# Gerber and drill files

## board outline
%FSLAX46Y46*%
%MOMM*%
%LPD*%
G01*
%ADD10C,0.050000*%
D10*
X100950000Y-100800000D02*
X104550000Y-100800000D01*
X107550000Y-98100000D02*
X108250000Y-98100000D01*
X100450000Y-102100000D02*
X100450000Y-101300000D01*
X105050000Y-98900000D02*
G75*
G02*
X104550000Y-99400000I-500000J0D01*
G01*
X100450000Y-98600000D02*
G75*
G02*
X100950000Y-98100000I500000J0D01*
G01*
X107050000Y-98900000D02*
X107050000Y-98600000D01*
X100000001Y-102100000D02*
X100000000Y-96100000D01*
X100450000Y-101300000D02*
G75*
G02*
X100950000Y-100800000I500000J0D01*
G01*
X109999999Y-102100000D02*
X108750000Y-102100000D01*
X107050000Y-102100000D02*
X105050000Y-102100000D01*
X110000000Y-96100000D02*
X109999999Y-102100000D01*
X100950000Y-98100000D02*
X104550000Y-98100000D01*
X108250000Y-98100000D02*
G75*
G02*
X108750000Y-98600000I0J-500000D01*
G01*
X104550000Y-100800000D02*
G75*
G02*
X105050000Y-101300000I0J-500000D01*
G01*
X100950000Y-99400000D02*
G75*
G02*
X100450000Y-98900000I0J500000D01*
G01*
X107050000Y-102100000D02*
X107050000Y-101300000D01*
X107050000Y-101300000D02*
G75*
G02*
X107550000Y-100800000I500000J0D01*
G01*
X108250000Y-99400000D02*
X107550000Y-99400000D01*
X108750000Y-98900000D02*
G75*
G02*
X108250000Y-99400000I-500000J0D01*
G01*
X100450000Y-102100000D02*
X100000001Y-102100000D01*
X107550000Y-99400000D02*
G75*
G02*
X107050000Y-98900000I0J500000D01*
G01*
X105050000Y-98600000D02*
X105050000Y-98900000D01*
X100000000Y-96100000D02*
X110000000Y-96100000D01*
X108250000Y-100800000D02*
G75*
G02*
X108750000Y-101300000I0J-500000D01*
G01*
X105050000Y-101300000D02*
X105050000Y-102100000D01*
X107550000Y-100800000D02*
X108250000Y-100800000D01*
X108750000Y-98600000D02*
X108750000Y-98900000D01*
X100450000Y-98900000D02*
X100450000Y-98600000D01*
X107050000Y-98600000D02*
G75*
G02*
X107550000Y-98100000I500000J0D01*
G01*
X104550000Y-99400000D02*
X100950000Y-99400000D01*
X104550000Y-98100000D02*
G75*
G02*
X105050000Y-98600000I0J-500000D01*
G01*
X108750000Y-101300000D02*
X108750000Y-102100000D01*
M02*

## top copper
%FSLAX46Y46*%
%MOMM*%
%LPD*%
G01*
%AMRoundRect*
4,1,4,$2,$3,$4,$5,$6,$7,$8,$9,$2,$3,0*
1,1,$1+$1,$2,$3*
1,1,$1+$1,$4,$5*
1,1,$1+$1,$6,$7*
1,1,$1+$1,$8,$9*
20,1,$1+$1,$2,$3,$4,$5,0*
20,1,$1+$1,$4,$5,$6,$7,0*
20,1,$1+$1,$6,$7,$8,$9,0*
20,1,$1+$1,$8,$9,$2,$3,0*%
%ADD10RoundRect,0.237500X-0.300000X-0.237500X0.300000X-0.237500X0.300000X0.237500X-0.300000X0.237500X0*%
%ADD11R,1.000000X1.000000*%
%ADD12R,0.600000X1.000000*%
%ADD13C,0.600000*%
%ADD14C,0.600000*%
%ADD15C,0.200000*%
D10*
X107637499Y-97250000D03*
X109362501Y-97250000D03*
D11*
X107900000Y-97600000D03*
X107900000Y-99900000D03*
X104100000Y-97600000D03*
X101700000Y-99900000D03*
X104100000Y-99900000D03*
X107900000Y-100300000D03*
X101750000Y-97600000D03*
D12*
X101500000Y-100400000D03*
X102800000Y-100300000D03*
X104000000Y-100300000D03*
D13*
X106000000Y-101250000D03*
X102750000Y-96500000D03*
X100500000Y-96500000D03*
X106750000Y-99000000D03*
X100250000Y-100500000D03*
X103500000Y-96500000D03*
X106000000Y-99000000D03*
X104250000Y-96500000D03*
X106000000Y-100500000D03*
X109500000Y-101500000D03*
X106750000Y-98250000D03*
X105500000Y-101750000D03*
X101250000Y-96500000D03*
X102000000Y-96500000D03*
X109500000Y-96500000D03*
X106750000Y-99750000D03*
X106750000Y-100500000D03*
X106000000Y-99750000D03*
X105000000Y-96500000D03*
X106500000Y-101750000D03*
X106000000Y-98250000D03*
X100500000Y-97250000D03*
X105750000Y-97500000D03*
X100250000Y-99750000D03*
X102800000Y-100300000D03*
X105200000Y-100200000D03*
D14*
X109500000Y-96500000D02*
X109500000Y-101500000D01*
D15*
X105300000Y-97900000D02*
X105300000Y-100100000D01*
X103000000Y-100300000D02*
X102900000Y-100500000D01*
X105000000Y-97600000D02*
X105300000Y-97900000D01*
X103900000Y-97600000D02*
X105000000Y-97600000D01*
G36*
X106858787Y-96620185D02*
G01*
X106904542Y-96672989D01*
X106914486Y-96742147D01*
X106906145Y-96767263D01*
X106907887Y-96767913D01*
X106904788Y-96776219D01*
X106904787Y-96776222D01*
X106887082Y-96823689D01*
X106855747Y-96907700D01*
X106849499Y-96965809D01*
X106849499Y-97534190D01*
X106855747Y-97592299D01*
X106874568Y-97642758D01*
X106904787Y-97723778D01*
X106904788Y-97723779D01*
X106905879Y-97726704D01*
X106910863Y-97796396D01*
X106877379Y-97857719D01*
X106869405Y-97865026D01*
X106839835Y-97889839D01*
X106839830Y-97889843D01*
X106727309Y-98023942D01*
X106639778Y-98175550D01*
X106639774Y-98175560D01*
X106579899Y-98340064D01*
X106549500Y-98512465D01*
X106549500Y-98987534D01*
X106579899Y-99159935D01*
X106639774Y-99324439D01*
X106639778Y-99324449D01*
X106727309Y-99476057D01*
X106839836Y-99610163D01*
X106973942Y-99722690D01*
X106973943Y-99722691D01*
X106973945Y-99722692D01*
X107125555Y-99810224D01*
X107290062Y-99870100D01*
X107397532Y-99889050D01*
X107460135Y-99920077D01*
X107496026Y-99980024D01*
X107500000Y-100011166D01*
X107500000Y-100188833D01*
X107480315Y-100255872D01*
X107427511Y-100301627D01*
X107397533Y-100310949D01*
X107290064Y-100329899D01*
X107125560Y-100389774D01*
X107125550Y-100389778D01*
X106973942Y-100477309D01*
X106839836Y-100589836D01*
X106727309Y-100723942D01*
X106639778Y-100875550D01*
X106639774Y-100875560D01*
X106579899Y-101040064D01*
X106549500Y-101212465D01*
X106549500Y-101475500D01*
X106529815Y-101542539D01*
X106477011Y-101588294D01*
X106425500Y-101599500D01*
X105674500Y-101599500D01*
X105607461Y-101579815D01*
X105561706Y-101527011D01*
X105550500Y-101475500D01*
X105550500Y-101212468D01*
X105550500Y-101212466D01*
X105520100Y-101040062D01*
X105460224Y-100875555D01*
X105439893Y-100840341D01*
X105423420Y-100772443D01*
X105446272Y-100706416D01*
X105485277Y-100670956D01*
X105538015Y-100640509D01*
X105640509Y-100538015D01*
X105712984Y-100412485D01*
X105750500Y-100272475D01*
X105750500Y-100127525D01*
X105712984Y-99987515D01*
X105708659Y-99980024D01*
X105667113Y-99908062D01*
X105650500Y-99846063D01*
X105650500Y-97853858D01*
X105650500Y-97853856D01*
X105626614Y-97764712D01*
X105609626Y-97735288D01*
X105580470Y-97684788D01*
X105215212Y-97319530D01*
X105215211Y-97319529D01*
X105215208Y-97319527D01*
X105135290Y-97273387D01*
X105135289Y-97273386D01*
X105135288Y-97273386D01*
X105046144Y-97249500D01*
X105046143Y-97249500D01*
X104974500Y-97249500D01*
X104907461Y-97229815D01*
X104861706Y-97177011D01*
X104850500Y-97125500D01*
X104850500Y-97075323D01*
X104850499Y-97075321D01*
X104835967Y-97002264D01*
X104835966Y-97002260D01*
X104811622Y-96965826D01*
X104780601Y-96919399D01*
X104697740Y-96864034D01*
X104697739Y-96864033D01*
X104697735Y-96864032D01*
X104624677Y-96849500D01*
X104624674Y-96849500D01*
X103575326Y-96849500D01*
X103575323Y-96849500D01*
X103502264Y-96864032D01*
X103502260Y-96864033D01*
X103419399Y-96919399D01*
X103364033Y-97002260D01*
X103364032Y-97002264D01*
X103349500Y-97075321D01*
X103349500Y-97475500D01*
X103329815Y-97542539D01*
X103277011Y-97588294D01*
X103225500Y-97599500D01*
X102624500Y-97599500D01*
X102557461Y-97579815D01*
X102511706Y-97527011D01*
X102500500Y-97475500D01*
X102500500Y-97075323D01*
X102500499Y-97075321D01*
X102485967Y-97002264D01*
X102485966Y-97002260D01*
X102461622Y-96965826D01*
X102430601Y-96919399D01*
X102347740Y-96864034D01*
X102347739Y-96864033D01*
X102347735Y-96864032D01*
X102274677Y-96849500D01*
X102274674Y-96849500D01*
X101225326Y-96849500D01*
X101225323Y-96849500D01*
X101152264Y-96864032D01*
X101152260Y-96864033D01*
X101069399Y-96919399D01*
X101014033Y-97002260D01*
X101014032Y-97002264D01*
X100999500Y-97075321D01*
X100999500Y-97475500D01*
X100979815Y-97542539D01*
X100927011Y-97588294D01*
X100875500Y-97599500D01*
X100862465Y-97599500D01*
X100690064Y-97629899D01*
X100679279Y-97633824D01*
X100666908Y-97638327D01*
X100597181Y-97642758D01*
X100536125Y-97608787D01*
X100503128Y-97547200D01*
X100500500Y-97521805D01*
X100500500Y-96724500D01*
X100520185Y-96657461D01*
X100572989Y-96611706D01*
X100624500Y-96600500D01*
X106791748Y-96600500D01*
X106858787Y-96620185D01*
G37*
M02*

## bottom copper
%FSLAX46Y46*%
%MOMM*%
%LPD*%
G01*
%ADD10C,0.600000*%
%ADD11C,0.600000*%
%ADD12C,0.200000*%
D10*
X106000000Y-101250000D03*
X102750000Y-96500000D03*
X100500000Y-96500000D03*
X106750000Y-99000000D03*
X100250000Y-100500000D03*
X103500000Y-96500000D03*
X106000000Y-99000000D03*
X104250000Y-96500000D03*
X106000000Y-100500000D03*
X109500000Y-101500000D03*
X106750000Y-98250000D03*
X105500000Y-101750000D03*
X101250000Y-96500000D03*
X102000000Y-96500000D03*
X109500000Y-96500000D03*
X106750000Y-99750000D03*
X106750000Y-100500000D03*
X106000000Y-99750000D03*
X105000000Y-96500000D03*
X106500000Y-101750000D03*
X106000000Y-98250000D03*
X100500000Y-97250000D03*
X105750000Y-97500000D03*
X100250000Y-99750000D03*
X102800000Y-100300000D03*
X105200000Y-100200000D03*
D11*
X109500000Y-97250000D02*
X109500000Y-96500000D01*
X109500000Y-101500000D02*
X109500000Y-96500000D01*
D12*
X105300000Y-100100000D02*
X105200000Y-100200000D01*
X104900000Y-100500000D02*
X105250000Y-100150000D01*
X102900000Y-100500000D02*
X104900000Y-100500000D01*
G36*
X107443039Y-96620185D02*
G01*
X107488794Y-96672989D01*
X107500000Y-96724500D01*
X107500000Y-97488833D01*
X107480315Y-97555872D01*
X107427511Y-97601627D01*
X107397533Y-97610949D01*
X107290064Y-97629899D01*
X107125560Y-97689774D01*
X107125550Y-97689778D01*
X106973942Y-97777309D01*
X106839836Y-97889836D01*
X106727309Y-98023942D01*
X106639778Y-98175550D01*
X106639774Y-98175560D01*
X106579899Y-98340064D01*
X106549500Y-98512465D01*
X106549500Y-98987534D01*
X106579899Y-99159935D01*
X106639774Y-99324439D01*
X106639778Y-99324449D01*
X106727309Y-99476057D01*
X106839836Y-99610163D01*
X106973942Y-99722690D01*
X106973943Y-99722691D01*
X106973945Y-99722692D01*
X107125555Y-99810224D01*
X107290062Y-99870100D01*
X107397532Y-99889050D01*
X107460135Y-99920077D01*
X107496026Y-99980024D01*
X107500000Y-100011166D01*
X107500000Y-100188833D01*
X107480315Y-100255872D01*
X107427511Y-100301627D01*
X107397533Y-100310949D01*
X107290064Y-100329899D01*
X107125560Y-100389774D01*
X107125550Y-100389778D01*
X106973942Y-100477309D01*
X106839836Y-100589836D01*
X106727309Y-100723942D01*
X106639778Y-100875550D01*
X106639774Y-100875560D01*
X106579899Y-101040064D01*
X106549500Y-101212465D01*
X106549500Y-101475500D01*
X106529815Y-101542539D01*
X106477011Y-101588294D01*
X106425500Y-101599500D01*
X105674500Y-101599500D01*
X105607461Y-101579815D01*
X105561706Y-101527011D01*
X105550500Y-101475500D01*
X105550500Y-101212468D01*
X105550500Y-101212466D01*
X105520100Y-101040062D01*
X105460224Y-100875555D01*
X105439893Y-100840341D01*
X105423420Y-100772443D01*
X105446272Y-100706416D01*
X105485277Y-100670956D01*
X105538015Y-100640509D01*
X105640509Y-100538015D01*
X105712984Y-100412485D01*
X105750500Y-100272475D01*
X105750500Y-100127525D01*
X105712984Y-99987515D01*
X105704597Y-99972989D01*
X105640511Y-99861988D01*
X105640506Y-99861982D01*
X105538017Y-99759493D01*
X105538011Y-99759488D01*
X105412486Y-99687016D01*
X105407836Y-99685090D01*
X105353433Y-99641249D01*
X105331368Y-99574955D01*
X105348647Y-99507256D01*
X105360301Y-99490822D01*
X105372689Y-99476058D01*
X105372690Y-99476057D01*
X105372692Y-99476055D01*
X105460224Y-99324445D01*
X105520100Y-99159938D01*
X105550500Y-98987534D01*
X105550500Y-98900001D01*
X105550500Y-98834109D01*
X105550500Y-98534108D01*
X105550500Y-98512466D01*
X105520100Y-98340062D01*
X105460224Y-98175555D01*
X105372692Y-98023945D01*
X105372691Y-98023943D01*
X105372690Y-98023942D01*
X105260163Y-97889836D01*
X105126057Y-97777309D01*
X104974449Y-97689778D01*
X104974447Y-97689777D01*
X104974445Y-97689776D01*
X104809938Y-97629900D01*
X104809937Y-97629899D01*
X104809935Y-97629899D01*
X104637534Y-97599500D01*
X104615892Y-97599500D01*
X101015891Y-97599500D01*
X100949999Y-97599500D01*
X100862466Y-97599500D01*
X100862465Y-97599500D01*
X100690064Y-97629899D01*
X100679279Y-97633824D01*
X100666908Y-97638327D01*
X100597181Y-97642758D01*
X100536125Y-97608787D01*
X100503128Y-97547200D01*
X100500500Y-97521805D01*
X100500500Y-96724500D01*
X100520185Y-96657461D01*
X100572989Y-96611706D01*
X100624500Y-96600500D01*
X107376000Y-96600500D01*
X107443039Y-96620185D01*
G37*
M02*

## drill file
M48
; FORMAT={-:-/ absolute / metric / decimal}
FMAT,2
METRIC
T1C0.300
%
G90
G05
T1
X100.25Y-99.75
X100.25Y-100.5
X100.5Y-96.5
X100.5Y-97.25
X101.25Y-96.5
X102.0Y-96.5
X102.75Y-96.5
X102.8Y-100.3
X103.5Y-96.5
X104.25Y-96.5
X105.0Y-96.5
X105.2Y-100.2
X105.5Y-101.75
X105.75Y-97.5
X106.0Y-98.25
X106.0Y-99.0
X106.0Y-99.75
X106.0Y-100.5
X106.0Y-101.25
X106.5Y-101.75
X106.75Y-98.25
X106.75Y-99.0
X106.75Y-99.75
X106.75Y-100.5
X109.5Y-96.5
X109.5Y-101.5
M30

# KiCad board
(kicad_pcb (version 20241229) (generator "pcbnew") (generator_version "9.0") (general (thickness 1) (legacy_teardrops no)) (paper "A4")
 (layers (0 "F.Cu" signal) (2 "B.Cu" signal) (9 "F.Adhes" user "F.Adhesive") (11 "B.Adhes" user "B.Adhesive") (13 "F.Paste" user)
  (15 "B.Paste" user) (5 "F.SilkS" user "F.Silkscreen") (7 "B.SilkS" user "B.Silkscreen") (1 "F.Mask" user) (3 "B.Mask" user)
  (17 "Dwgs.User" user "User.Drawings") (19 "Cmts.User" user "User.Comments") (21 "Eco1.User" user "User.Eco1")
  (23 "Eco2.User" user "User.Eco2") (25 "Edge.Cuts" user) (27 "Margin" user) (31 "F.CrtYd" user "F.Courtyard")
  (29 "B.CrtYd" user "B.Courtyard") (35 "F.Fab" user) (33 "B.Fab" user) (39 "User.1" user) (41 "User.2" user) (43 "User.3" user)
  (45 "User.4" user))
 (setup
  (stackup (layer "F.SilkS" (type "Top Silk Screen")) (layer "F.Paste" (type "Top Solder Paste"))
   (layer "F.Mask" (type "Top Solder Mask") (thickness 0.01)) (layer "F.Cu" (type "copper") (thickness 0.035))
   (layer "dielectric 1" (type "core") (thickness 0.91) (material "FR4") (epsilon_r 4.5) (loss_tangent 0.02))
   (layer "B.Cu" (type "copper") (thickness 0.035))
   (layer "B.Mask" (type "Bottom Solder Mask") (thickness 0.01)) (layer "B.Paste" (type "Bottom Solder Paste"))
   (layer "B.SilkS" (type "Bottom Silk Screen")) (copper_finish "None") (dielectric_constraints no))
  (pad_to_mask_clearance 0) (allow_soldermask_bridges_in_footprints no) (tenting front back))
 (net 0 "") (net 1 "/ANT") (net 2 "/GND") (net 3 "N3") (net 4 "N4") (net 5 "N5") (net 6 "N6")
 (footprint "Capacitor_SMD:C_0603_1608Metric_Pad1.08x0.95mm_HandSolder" (layer "F.Cu") (at 108.5 97.25)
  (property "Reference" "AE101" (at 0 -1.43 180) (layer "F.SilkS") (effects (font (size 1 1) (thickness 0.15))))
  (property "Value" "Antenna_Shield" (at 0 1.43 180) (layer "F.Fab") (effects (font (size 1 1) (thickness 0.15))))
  (pad "1" smd roundrect (at -0.862501 0) (size 1.075 0.95) (layers "F.Cu" "F.Mask" "F.Paste") (roundrect_rratio 0.25) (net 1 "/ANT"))
  (pad "2" smd roundrect (at 0.862501 0) (size 1.075 0.95) (layers "F.Cu" "F.Mask" "F.Paste") (roundrect_rratio 0.25) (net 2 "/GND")))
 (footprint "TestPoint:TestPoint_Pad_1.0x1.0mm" (layer "F.Cu") (at 107.9 97.6)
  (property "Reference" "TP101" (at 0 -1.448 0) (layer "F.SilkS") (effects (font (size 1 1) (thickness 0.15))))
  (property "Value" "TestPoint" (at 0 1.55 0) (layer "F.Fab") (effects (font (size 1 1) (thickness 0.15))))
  (pad "1" smd rect (at 0 0) (size 1 1) (layers "F.Cu" "F.Mask") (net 1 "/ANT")))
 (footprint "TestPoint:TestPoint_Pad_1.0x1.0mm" (layer "F.Cu") (at 107.9 99.9)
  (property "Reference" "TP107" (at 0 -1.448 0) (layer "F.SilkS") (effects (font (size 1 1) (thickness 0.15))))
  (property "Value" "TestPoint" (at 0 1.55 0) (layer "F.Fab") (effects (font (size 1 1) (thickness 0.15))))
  (pad "1" smd rect (at 0 0) (size 1 1) (layers "F.Cu" "F.Mask") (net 2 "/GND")))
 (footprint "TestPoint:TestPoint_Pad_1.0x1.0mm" (layer "F.Cu") (at 104.1 97.6 -90)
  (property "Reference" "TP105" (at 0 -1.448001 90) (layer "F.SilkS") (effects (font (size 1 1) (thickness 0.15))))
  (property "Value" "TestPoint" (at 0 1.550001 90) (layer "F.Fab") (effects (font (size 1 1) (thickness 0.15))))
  (pad "1" smd rect (at 0 0 270) (size 1 1) (layers "F.Cu" "F.Mask") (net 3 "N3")))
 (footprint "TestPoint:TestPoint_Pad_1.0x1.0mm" (layer "F.Cu") (at 101.7 99.9)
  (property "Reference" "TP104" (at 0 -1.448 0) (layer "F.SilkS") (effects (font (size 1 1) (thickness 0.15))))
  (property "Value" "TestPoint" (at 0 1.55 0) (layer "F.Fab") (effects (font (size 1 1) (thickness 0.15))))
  (pad "1" smd rect (at 0 0) (size 1 1) (layers "F.Cu" "F.Mask") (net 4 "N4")))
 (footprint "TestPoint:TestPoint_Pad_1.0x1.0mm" (layer "F.Cu") (at 104.1 99.9)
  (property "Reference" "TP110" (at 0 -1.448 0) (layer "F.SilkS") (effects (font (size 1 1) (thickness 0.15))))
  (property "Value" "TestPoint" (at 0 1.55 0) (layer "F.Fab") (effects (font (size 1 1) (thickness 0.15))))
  (pad "1" smd rect (at 0 0) (size 1 1) (layers "F.Cu" "F.Mask") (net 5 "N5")))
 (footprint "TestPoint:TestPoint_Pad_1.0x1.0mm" (layer "F.Cu") (at 107.9 100.3)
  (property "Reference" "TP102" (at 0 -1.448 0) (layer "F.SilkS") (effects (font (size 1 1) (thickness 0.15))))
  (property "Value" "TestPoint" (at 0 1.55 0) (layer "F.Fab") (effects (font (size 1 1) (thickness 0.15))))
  (pad "1" smd rect (at 0 0) (size 1 1) (layers "F.Cu" "F.Mask") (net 2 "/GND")))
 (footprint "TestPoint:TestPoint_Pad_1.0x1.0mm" (layer "F.Cu") (at 101.7 97.6)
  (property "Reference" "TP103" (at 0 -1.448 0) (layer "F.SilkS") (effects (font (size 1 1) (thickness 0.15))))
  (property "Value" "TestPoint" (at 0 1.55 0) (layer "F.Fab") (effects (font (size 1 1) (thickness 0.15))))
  (pad "1" smd rect (at 0.05 0) (size 1 1) (layers "F.Cu" "F.Mask") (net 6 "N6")))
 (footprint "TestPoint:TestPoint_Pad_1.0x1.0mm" (layer "F.Cu") (at 101.5 100.4)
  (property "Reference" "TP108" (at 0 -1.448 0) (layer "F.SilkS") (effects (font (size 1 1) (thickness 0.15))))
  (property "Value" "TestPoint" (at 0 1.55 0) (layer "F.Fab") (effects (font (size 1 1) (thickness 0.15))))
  (pad "1" smd rect (at 0 0) (size 0.6 1) (layers "F.Cu" "F.Mask") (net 4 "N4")))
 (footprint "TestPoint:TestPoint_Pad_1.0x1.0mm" (layer "F.Cu") (at 102.7 100.3)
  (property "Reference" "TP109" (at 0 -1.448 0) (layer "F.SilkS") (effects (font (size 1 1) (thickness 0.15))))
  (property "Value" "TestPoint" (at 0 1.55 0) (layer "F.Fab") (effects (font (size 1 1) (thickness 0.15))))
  (pad "1" smd rect (at 0.1 0) (size 0.6 1) (layers "F.Cu" "F.Mask") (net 3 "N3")))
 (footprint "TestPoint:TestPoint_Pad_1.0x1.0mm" (layer "F.Cu") (at 104 100.3)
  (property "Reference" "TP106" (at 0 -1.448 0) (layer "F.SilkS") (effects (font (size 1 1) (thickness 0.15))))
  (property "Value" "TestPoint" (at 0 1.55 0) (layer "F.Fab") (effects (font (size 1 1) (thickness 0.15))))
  (pad "1" smd rect (at 0 0) (size 0.6 1) (layers "F.Cu" "F.Mask") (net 5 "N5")))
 (gr_line (start 100.95 100.8) (end 104.55 100.8) (stroke (width 0.05) (type default)) (layer "Edge.Cuts"))
 (gr_line (start 107.55 98.1) (end 108.25 98.1) (stroke (width 0.05) (type default)) (layer "Edge.Cuts"))
 (gr_line (start 100.45 102.1) (end 100.45 101.3) (stroke (width 0.05) (type default)) (layer "Edge.Cuts"))
 (gr_arc (start 105.05 98.9) (mid 104.903553 99.253553) (end 104.55 99.4) (stroke (width 0.05) (type default)) (layer "Edge.Cuts"))
 (gr_arc (start 100.45 98.6) (mid 100.596447 98.246447) (end 100.95 98.1) (stroke (width 0.05) (type default)) (layer "Edge.Cuts"))
 (gr_line (start 107.05 98.9) (end 107.05 98.6) (stroke (width 0.05) (type default)) (layer "Edge.Cuts"))
 (gr_line (start 100.000001 102.1) (end 100 96.1) (stroke (width 0.05) (type default)) (layer "Edge.Cuts"))
 (gr_arc (start 100.45 101.3) (mid 100.596447 100.946447) (end 100.95 100.8) (stroke (width 0.05) (type default)) (layer "Edge.Cuts"))
 (gr_line (start 109.999999 102.1) (end 108.75 102.1) (stroke (width 0.05) (type default)) (layer "Edge.Cuts"))
 (gr_line (start 107.05 102.1) (end 105.05 102.1) (stroke (width 0.05) (type default)) (layer "Edge.Cuts"))
 (gr_line (start 110 96.1) (end 109.999999 102.1) (stroke (width 0.05) (type default)) (layer "Edge.Cuts"))
 (gr_line (start 100.95 98.1) (end 104.55 98.1) (stroke (width 0.05) (type default)) (layer "Edge.Cuts"))
 (gr_arc (start 108.25 98.1) (mid 108.603553 98.246447) (end 108.75 98.6) (stroke (width 0.05) (type default)) (layer "Edge.Cuts"))
 (gr_arc (start 104.55 100.8) (mid 104.903553 100.946447) (end 105.05 101.3) (stroke (width 0.05) (type default)) (layer "Edge.Cuts"))
 (gr_arc (start 100.95 99.4) (mid 100.596447 99.253553) (end 100.45 98.9) (stroke (width 0.05) (type default)) (layer "Edge.Cuts"))
 (gr_line (start 107.05 102.1) (end 107.05 101.3) (stroke (width 0.05) (type default)) (layer "Edge.Cuts"))
 (gr_arc (start 107.05 101.3) (mid 107.196447 100.946447) (end 107.55 100.8) (stroke (width 0.05) (type default)) (layer "Edge.Cuts"))
 (gr_line (start 108.25 99.4) (end 107.55 99.4) (stroke (width 0.05) (type default)) (layer "Edge.Cuts"))
 (gr_arc (start 108.75 98.9) (mid 108.603553 99.253553) (end 108.25 99.4) (stroke (width 0.05) (type default)) (layer "Edge.Cuts"))
 (gr_line (start 100.45 102.1) (end 100.000001 102.1) (stroke (width 0.05) (type default)) (layer "Edge.Cuts"))
 (gr_arc (start 107.55 99.4) (mid 107.196447 99.253553) (end 107.05 98.9) (stroke (width 0.05) (type default)) (layer "Edge.Cuts"))
 (gr_line (start 105.05 98.6) (end 105.05 98.9) (stroke (width 0.05) (type default)) (layer "Edge.Cuts"))
 (gr_line (start 100 96.1) (end 110 96.1) (stroke (width 0.05) (type default)) (layer "Edge.Cuts"))
 (gr_arc (start 108.25 100.8) (mid 108.603553 100.946447) (end 108.75 101.3) (stroke (width 0.05) (type default)) (layer "Edge.Cuts"))
 (gr_line (start 105.05 101.3) (end 105.05 102.1) (stroke (width 0.05) (type default)) (layer "Edge.Cuts"))
 (gr_line (start 107.55 100.8) (end 108.25 100.8) (stroke (width 0.05) (type default)) (layer "Edge.Cuts"))
 (gr_line (start 108.75 98.6) (end 108.75 98.9) (stroke (width 0.05) (type default)) (layer "Edge.Cuts"))
 (gr_line (start 100.45 98.9) (end 100.45 98.6) (stroke (width 0.05) (type default)) (layer "Edge.Cuts"))
 (gr_arc (start 107.05 98.6) (mid 107.196447 98.246447) (end 107.55 98.1) (stroke (width 0.05) (type default)) (layer "Edge.Cuts"))
 (gr_line (start 104.55 99.4) (end 100.95 99.4) (stroke (width 0.05) (type default)) (layer "Edge.Cuts"))
 (gr_arc (start 104.55 98.1) (mid 104.903553 98.246447) (end 105.05 98.6) (stroke (width 0.05) (type default)) (layer "Edge.Cuts"))
 (gr_line (start 108.75 101.3) (end 108.75 102.1) (stroke (width 0.05) (type default)) (layer "Edge.Cuts"))
 (segment (start 109.5 96.5) (end 109.5 101.5) (width 0.6) (layer "F.Cu") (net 2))
 (via (at 106 101.25) (size 0.6) (drill 0.3) (layers "F.Cu" "B.Cu") (free yes) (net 2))
 (via (at 102.75 96.5) (size 0.6) (drill 0.3) (layers "F.Cu" "B.Cu") (free yes) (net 2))
 (via (at 100.5 96.5) (size 0.6) (drill 0.3) (layers "F.Cu" "B.Cu") (free yes) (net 2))
 (via (at 106.75 99) (size 0.6) (drill 0.3) (layers "F.Cu" "B.Cu") (free yes) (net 2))
 (via (at 100.25 100.5) (size 0.6) (drill 0.3) (layers "F.Cu" "B.Cu") (free yes) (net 2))
 (via (at 103.5 96.5) (size 0.6) (drill 0.3) (layers "F.Cu" "B.Cu") (free yes) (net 2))
 (via (at 106 99) (size 0.6) (drill 0.3) (layers "F.Cu" "B.Cu") (free yes) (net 2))
 (via (at 104.25 96.5) (size 0.6) (drill 0.3) (layers "F.Cu" "B.Cu") (free yes) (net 2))
 (via (at 106 100.5) (size 0.6) (drill 0.3) (layers "F.Cu" "B.Cu") (free yes) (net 2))
 (via (at 109.5 101.5) (size 0.6) (drill 0.3) (layers "F.Cu" "B.Cu") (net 2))
 (via (at 106.75 98.25) (size 0.6) (drill 0.3) (layers "F.Cu" "B.Cu") (free yes) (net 2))
 (via (at 105.5 101.75) (size 0.6) (drill 0.3) (layers "F.Cu" "B.Cu") (free yes) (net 2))
 (via (at 101.25 96.5) (size 0.6) (drill 0.3) (layers "F.Cu" "B.Cu") (free yes) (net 2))
 (via (at 102 96.5) (size 0.6) (drill 0.3) (layers "F.Cu" "B.Cu") (free yes) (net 2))
 (via (at 109.5 96.5) (size 0.6) (drill 0.3) (layers "F.Cu" "B.Cu") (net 2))
 (via (at 106.75 99.75) (size 0.6) (drill 0.3) (layers "F.Cu" "B.Cu") (free yes) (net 2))
 (via (at 106.75 100.5) (size 0.6) (drill 0.3) (layers "F.Cu" "B.Cu") (free yes) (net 2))
 (via (at 106 99.75) (size 0.6) (drill 0.3) (layers "F.Cu" "B.Cu") (free yes) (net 2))
 (via (at 105 96.5) (size 0.6) (drill 0.3) (layers "F.Cu" "B.Cu") (free yes) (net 2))
 (via (at 106.5 101.75) (size 0.6) (drill 0.3) (layers "F.Cu" "B.Cu") (free yes) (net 2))
 (via (at 106 98.25) (size 0.6) (drill 0.3) (layers "F.Cu" "B.Cu") (free yes) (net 2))
 (via (at 100.5 97.25) (size 0.6) (drill 0.3) (layers "F.Cu" "B.Cu") (free yes) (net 2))
 (via (at 105.75 97.5) (size 0.6) (drill 0.3) (layers "F.Cu" "B.Cu") (free yes) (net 2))
 (via (at 100.25 99.75) (size 0.6) (drill 0.3) (layers "F.Cu" "B.Cu") (free yes) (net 2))
 (segment (start 109.5 97.25) (end 109.5 96.5) (width 0.6) (layer "B.Cu") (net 2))
 (segment (start 109.5 101.5) (end 109.5 96.5) (width 0.6) (layer "B.Cu") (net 2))
 (segment (start 105.3 97.9) (end 105.3 100.1) (width 0.2) (layer "F.Cu") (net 3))
 (segment (start 103 100.3) (end 102.9 100.5) (width 0.2) (layer "F.Cu") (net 3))
 (segment (start 105 97.6) (end 105.3 97.9) (width 0.2) (layer "F.Cu") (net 3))
 (segment (start 103.9 97.6) (end 105 97.6) (width 0.2) (layer "F.Cu") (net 3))
 (via (at 102.8 100.3) (size 0.6) (drill 0.3) (layers "F.Cu" "B.Cu") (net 3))
 (via (at 105.2 100.2) (size 0.6) (drill 0.3) (layers "F.Cu" "B.Cu") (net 3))
 (segment (start 105.3 100.1) (end 105.2 100.2) (width 0.2) (layer "B.Cu") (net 3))
 (segment (start 104.9 100.5) (end 105.25 100.15) (width 0.2) (layer "B.Cu") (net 3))
 (segment (start 102.9 100.5) (end 104.9 100.5) (width 0.2) (layer "B.Cu") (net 3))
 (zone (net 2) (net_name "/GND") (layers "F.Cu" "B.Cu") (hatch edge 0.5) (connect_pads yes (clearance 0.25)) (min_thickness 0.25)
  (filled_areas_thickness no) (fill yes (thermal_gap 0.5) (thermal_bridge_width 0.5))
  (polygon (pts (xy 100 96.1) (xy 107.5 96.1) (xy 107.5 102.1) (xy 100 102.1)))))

